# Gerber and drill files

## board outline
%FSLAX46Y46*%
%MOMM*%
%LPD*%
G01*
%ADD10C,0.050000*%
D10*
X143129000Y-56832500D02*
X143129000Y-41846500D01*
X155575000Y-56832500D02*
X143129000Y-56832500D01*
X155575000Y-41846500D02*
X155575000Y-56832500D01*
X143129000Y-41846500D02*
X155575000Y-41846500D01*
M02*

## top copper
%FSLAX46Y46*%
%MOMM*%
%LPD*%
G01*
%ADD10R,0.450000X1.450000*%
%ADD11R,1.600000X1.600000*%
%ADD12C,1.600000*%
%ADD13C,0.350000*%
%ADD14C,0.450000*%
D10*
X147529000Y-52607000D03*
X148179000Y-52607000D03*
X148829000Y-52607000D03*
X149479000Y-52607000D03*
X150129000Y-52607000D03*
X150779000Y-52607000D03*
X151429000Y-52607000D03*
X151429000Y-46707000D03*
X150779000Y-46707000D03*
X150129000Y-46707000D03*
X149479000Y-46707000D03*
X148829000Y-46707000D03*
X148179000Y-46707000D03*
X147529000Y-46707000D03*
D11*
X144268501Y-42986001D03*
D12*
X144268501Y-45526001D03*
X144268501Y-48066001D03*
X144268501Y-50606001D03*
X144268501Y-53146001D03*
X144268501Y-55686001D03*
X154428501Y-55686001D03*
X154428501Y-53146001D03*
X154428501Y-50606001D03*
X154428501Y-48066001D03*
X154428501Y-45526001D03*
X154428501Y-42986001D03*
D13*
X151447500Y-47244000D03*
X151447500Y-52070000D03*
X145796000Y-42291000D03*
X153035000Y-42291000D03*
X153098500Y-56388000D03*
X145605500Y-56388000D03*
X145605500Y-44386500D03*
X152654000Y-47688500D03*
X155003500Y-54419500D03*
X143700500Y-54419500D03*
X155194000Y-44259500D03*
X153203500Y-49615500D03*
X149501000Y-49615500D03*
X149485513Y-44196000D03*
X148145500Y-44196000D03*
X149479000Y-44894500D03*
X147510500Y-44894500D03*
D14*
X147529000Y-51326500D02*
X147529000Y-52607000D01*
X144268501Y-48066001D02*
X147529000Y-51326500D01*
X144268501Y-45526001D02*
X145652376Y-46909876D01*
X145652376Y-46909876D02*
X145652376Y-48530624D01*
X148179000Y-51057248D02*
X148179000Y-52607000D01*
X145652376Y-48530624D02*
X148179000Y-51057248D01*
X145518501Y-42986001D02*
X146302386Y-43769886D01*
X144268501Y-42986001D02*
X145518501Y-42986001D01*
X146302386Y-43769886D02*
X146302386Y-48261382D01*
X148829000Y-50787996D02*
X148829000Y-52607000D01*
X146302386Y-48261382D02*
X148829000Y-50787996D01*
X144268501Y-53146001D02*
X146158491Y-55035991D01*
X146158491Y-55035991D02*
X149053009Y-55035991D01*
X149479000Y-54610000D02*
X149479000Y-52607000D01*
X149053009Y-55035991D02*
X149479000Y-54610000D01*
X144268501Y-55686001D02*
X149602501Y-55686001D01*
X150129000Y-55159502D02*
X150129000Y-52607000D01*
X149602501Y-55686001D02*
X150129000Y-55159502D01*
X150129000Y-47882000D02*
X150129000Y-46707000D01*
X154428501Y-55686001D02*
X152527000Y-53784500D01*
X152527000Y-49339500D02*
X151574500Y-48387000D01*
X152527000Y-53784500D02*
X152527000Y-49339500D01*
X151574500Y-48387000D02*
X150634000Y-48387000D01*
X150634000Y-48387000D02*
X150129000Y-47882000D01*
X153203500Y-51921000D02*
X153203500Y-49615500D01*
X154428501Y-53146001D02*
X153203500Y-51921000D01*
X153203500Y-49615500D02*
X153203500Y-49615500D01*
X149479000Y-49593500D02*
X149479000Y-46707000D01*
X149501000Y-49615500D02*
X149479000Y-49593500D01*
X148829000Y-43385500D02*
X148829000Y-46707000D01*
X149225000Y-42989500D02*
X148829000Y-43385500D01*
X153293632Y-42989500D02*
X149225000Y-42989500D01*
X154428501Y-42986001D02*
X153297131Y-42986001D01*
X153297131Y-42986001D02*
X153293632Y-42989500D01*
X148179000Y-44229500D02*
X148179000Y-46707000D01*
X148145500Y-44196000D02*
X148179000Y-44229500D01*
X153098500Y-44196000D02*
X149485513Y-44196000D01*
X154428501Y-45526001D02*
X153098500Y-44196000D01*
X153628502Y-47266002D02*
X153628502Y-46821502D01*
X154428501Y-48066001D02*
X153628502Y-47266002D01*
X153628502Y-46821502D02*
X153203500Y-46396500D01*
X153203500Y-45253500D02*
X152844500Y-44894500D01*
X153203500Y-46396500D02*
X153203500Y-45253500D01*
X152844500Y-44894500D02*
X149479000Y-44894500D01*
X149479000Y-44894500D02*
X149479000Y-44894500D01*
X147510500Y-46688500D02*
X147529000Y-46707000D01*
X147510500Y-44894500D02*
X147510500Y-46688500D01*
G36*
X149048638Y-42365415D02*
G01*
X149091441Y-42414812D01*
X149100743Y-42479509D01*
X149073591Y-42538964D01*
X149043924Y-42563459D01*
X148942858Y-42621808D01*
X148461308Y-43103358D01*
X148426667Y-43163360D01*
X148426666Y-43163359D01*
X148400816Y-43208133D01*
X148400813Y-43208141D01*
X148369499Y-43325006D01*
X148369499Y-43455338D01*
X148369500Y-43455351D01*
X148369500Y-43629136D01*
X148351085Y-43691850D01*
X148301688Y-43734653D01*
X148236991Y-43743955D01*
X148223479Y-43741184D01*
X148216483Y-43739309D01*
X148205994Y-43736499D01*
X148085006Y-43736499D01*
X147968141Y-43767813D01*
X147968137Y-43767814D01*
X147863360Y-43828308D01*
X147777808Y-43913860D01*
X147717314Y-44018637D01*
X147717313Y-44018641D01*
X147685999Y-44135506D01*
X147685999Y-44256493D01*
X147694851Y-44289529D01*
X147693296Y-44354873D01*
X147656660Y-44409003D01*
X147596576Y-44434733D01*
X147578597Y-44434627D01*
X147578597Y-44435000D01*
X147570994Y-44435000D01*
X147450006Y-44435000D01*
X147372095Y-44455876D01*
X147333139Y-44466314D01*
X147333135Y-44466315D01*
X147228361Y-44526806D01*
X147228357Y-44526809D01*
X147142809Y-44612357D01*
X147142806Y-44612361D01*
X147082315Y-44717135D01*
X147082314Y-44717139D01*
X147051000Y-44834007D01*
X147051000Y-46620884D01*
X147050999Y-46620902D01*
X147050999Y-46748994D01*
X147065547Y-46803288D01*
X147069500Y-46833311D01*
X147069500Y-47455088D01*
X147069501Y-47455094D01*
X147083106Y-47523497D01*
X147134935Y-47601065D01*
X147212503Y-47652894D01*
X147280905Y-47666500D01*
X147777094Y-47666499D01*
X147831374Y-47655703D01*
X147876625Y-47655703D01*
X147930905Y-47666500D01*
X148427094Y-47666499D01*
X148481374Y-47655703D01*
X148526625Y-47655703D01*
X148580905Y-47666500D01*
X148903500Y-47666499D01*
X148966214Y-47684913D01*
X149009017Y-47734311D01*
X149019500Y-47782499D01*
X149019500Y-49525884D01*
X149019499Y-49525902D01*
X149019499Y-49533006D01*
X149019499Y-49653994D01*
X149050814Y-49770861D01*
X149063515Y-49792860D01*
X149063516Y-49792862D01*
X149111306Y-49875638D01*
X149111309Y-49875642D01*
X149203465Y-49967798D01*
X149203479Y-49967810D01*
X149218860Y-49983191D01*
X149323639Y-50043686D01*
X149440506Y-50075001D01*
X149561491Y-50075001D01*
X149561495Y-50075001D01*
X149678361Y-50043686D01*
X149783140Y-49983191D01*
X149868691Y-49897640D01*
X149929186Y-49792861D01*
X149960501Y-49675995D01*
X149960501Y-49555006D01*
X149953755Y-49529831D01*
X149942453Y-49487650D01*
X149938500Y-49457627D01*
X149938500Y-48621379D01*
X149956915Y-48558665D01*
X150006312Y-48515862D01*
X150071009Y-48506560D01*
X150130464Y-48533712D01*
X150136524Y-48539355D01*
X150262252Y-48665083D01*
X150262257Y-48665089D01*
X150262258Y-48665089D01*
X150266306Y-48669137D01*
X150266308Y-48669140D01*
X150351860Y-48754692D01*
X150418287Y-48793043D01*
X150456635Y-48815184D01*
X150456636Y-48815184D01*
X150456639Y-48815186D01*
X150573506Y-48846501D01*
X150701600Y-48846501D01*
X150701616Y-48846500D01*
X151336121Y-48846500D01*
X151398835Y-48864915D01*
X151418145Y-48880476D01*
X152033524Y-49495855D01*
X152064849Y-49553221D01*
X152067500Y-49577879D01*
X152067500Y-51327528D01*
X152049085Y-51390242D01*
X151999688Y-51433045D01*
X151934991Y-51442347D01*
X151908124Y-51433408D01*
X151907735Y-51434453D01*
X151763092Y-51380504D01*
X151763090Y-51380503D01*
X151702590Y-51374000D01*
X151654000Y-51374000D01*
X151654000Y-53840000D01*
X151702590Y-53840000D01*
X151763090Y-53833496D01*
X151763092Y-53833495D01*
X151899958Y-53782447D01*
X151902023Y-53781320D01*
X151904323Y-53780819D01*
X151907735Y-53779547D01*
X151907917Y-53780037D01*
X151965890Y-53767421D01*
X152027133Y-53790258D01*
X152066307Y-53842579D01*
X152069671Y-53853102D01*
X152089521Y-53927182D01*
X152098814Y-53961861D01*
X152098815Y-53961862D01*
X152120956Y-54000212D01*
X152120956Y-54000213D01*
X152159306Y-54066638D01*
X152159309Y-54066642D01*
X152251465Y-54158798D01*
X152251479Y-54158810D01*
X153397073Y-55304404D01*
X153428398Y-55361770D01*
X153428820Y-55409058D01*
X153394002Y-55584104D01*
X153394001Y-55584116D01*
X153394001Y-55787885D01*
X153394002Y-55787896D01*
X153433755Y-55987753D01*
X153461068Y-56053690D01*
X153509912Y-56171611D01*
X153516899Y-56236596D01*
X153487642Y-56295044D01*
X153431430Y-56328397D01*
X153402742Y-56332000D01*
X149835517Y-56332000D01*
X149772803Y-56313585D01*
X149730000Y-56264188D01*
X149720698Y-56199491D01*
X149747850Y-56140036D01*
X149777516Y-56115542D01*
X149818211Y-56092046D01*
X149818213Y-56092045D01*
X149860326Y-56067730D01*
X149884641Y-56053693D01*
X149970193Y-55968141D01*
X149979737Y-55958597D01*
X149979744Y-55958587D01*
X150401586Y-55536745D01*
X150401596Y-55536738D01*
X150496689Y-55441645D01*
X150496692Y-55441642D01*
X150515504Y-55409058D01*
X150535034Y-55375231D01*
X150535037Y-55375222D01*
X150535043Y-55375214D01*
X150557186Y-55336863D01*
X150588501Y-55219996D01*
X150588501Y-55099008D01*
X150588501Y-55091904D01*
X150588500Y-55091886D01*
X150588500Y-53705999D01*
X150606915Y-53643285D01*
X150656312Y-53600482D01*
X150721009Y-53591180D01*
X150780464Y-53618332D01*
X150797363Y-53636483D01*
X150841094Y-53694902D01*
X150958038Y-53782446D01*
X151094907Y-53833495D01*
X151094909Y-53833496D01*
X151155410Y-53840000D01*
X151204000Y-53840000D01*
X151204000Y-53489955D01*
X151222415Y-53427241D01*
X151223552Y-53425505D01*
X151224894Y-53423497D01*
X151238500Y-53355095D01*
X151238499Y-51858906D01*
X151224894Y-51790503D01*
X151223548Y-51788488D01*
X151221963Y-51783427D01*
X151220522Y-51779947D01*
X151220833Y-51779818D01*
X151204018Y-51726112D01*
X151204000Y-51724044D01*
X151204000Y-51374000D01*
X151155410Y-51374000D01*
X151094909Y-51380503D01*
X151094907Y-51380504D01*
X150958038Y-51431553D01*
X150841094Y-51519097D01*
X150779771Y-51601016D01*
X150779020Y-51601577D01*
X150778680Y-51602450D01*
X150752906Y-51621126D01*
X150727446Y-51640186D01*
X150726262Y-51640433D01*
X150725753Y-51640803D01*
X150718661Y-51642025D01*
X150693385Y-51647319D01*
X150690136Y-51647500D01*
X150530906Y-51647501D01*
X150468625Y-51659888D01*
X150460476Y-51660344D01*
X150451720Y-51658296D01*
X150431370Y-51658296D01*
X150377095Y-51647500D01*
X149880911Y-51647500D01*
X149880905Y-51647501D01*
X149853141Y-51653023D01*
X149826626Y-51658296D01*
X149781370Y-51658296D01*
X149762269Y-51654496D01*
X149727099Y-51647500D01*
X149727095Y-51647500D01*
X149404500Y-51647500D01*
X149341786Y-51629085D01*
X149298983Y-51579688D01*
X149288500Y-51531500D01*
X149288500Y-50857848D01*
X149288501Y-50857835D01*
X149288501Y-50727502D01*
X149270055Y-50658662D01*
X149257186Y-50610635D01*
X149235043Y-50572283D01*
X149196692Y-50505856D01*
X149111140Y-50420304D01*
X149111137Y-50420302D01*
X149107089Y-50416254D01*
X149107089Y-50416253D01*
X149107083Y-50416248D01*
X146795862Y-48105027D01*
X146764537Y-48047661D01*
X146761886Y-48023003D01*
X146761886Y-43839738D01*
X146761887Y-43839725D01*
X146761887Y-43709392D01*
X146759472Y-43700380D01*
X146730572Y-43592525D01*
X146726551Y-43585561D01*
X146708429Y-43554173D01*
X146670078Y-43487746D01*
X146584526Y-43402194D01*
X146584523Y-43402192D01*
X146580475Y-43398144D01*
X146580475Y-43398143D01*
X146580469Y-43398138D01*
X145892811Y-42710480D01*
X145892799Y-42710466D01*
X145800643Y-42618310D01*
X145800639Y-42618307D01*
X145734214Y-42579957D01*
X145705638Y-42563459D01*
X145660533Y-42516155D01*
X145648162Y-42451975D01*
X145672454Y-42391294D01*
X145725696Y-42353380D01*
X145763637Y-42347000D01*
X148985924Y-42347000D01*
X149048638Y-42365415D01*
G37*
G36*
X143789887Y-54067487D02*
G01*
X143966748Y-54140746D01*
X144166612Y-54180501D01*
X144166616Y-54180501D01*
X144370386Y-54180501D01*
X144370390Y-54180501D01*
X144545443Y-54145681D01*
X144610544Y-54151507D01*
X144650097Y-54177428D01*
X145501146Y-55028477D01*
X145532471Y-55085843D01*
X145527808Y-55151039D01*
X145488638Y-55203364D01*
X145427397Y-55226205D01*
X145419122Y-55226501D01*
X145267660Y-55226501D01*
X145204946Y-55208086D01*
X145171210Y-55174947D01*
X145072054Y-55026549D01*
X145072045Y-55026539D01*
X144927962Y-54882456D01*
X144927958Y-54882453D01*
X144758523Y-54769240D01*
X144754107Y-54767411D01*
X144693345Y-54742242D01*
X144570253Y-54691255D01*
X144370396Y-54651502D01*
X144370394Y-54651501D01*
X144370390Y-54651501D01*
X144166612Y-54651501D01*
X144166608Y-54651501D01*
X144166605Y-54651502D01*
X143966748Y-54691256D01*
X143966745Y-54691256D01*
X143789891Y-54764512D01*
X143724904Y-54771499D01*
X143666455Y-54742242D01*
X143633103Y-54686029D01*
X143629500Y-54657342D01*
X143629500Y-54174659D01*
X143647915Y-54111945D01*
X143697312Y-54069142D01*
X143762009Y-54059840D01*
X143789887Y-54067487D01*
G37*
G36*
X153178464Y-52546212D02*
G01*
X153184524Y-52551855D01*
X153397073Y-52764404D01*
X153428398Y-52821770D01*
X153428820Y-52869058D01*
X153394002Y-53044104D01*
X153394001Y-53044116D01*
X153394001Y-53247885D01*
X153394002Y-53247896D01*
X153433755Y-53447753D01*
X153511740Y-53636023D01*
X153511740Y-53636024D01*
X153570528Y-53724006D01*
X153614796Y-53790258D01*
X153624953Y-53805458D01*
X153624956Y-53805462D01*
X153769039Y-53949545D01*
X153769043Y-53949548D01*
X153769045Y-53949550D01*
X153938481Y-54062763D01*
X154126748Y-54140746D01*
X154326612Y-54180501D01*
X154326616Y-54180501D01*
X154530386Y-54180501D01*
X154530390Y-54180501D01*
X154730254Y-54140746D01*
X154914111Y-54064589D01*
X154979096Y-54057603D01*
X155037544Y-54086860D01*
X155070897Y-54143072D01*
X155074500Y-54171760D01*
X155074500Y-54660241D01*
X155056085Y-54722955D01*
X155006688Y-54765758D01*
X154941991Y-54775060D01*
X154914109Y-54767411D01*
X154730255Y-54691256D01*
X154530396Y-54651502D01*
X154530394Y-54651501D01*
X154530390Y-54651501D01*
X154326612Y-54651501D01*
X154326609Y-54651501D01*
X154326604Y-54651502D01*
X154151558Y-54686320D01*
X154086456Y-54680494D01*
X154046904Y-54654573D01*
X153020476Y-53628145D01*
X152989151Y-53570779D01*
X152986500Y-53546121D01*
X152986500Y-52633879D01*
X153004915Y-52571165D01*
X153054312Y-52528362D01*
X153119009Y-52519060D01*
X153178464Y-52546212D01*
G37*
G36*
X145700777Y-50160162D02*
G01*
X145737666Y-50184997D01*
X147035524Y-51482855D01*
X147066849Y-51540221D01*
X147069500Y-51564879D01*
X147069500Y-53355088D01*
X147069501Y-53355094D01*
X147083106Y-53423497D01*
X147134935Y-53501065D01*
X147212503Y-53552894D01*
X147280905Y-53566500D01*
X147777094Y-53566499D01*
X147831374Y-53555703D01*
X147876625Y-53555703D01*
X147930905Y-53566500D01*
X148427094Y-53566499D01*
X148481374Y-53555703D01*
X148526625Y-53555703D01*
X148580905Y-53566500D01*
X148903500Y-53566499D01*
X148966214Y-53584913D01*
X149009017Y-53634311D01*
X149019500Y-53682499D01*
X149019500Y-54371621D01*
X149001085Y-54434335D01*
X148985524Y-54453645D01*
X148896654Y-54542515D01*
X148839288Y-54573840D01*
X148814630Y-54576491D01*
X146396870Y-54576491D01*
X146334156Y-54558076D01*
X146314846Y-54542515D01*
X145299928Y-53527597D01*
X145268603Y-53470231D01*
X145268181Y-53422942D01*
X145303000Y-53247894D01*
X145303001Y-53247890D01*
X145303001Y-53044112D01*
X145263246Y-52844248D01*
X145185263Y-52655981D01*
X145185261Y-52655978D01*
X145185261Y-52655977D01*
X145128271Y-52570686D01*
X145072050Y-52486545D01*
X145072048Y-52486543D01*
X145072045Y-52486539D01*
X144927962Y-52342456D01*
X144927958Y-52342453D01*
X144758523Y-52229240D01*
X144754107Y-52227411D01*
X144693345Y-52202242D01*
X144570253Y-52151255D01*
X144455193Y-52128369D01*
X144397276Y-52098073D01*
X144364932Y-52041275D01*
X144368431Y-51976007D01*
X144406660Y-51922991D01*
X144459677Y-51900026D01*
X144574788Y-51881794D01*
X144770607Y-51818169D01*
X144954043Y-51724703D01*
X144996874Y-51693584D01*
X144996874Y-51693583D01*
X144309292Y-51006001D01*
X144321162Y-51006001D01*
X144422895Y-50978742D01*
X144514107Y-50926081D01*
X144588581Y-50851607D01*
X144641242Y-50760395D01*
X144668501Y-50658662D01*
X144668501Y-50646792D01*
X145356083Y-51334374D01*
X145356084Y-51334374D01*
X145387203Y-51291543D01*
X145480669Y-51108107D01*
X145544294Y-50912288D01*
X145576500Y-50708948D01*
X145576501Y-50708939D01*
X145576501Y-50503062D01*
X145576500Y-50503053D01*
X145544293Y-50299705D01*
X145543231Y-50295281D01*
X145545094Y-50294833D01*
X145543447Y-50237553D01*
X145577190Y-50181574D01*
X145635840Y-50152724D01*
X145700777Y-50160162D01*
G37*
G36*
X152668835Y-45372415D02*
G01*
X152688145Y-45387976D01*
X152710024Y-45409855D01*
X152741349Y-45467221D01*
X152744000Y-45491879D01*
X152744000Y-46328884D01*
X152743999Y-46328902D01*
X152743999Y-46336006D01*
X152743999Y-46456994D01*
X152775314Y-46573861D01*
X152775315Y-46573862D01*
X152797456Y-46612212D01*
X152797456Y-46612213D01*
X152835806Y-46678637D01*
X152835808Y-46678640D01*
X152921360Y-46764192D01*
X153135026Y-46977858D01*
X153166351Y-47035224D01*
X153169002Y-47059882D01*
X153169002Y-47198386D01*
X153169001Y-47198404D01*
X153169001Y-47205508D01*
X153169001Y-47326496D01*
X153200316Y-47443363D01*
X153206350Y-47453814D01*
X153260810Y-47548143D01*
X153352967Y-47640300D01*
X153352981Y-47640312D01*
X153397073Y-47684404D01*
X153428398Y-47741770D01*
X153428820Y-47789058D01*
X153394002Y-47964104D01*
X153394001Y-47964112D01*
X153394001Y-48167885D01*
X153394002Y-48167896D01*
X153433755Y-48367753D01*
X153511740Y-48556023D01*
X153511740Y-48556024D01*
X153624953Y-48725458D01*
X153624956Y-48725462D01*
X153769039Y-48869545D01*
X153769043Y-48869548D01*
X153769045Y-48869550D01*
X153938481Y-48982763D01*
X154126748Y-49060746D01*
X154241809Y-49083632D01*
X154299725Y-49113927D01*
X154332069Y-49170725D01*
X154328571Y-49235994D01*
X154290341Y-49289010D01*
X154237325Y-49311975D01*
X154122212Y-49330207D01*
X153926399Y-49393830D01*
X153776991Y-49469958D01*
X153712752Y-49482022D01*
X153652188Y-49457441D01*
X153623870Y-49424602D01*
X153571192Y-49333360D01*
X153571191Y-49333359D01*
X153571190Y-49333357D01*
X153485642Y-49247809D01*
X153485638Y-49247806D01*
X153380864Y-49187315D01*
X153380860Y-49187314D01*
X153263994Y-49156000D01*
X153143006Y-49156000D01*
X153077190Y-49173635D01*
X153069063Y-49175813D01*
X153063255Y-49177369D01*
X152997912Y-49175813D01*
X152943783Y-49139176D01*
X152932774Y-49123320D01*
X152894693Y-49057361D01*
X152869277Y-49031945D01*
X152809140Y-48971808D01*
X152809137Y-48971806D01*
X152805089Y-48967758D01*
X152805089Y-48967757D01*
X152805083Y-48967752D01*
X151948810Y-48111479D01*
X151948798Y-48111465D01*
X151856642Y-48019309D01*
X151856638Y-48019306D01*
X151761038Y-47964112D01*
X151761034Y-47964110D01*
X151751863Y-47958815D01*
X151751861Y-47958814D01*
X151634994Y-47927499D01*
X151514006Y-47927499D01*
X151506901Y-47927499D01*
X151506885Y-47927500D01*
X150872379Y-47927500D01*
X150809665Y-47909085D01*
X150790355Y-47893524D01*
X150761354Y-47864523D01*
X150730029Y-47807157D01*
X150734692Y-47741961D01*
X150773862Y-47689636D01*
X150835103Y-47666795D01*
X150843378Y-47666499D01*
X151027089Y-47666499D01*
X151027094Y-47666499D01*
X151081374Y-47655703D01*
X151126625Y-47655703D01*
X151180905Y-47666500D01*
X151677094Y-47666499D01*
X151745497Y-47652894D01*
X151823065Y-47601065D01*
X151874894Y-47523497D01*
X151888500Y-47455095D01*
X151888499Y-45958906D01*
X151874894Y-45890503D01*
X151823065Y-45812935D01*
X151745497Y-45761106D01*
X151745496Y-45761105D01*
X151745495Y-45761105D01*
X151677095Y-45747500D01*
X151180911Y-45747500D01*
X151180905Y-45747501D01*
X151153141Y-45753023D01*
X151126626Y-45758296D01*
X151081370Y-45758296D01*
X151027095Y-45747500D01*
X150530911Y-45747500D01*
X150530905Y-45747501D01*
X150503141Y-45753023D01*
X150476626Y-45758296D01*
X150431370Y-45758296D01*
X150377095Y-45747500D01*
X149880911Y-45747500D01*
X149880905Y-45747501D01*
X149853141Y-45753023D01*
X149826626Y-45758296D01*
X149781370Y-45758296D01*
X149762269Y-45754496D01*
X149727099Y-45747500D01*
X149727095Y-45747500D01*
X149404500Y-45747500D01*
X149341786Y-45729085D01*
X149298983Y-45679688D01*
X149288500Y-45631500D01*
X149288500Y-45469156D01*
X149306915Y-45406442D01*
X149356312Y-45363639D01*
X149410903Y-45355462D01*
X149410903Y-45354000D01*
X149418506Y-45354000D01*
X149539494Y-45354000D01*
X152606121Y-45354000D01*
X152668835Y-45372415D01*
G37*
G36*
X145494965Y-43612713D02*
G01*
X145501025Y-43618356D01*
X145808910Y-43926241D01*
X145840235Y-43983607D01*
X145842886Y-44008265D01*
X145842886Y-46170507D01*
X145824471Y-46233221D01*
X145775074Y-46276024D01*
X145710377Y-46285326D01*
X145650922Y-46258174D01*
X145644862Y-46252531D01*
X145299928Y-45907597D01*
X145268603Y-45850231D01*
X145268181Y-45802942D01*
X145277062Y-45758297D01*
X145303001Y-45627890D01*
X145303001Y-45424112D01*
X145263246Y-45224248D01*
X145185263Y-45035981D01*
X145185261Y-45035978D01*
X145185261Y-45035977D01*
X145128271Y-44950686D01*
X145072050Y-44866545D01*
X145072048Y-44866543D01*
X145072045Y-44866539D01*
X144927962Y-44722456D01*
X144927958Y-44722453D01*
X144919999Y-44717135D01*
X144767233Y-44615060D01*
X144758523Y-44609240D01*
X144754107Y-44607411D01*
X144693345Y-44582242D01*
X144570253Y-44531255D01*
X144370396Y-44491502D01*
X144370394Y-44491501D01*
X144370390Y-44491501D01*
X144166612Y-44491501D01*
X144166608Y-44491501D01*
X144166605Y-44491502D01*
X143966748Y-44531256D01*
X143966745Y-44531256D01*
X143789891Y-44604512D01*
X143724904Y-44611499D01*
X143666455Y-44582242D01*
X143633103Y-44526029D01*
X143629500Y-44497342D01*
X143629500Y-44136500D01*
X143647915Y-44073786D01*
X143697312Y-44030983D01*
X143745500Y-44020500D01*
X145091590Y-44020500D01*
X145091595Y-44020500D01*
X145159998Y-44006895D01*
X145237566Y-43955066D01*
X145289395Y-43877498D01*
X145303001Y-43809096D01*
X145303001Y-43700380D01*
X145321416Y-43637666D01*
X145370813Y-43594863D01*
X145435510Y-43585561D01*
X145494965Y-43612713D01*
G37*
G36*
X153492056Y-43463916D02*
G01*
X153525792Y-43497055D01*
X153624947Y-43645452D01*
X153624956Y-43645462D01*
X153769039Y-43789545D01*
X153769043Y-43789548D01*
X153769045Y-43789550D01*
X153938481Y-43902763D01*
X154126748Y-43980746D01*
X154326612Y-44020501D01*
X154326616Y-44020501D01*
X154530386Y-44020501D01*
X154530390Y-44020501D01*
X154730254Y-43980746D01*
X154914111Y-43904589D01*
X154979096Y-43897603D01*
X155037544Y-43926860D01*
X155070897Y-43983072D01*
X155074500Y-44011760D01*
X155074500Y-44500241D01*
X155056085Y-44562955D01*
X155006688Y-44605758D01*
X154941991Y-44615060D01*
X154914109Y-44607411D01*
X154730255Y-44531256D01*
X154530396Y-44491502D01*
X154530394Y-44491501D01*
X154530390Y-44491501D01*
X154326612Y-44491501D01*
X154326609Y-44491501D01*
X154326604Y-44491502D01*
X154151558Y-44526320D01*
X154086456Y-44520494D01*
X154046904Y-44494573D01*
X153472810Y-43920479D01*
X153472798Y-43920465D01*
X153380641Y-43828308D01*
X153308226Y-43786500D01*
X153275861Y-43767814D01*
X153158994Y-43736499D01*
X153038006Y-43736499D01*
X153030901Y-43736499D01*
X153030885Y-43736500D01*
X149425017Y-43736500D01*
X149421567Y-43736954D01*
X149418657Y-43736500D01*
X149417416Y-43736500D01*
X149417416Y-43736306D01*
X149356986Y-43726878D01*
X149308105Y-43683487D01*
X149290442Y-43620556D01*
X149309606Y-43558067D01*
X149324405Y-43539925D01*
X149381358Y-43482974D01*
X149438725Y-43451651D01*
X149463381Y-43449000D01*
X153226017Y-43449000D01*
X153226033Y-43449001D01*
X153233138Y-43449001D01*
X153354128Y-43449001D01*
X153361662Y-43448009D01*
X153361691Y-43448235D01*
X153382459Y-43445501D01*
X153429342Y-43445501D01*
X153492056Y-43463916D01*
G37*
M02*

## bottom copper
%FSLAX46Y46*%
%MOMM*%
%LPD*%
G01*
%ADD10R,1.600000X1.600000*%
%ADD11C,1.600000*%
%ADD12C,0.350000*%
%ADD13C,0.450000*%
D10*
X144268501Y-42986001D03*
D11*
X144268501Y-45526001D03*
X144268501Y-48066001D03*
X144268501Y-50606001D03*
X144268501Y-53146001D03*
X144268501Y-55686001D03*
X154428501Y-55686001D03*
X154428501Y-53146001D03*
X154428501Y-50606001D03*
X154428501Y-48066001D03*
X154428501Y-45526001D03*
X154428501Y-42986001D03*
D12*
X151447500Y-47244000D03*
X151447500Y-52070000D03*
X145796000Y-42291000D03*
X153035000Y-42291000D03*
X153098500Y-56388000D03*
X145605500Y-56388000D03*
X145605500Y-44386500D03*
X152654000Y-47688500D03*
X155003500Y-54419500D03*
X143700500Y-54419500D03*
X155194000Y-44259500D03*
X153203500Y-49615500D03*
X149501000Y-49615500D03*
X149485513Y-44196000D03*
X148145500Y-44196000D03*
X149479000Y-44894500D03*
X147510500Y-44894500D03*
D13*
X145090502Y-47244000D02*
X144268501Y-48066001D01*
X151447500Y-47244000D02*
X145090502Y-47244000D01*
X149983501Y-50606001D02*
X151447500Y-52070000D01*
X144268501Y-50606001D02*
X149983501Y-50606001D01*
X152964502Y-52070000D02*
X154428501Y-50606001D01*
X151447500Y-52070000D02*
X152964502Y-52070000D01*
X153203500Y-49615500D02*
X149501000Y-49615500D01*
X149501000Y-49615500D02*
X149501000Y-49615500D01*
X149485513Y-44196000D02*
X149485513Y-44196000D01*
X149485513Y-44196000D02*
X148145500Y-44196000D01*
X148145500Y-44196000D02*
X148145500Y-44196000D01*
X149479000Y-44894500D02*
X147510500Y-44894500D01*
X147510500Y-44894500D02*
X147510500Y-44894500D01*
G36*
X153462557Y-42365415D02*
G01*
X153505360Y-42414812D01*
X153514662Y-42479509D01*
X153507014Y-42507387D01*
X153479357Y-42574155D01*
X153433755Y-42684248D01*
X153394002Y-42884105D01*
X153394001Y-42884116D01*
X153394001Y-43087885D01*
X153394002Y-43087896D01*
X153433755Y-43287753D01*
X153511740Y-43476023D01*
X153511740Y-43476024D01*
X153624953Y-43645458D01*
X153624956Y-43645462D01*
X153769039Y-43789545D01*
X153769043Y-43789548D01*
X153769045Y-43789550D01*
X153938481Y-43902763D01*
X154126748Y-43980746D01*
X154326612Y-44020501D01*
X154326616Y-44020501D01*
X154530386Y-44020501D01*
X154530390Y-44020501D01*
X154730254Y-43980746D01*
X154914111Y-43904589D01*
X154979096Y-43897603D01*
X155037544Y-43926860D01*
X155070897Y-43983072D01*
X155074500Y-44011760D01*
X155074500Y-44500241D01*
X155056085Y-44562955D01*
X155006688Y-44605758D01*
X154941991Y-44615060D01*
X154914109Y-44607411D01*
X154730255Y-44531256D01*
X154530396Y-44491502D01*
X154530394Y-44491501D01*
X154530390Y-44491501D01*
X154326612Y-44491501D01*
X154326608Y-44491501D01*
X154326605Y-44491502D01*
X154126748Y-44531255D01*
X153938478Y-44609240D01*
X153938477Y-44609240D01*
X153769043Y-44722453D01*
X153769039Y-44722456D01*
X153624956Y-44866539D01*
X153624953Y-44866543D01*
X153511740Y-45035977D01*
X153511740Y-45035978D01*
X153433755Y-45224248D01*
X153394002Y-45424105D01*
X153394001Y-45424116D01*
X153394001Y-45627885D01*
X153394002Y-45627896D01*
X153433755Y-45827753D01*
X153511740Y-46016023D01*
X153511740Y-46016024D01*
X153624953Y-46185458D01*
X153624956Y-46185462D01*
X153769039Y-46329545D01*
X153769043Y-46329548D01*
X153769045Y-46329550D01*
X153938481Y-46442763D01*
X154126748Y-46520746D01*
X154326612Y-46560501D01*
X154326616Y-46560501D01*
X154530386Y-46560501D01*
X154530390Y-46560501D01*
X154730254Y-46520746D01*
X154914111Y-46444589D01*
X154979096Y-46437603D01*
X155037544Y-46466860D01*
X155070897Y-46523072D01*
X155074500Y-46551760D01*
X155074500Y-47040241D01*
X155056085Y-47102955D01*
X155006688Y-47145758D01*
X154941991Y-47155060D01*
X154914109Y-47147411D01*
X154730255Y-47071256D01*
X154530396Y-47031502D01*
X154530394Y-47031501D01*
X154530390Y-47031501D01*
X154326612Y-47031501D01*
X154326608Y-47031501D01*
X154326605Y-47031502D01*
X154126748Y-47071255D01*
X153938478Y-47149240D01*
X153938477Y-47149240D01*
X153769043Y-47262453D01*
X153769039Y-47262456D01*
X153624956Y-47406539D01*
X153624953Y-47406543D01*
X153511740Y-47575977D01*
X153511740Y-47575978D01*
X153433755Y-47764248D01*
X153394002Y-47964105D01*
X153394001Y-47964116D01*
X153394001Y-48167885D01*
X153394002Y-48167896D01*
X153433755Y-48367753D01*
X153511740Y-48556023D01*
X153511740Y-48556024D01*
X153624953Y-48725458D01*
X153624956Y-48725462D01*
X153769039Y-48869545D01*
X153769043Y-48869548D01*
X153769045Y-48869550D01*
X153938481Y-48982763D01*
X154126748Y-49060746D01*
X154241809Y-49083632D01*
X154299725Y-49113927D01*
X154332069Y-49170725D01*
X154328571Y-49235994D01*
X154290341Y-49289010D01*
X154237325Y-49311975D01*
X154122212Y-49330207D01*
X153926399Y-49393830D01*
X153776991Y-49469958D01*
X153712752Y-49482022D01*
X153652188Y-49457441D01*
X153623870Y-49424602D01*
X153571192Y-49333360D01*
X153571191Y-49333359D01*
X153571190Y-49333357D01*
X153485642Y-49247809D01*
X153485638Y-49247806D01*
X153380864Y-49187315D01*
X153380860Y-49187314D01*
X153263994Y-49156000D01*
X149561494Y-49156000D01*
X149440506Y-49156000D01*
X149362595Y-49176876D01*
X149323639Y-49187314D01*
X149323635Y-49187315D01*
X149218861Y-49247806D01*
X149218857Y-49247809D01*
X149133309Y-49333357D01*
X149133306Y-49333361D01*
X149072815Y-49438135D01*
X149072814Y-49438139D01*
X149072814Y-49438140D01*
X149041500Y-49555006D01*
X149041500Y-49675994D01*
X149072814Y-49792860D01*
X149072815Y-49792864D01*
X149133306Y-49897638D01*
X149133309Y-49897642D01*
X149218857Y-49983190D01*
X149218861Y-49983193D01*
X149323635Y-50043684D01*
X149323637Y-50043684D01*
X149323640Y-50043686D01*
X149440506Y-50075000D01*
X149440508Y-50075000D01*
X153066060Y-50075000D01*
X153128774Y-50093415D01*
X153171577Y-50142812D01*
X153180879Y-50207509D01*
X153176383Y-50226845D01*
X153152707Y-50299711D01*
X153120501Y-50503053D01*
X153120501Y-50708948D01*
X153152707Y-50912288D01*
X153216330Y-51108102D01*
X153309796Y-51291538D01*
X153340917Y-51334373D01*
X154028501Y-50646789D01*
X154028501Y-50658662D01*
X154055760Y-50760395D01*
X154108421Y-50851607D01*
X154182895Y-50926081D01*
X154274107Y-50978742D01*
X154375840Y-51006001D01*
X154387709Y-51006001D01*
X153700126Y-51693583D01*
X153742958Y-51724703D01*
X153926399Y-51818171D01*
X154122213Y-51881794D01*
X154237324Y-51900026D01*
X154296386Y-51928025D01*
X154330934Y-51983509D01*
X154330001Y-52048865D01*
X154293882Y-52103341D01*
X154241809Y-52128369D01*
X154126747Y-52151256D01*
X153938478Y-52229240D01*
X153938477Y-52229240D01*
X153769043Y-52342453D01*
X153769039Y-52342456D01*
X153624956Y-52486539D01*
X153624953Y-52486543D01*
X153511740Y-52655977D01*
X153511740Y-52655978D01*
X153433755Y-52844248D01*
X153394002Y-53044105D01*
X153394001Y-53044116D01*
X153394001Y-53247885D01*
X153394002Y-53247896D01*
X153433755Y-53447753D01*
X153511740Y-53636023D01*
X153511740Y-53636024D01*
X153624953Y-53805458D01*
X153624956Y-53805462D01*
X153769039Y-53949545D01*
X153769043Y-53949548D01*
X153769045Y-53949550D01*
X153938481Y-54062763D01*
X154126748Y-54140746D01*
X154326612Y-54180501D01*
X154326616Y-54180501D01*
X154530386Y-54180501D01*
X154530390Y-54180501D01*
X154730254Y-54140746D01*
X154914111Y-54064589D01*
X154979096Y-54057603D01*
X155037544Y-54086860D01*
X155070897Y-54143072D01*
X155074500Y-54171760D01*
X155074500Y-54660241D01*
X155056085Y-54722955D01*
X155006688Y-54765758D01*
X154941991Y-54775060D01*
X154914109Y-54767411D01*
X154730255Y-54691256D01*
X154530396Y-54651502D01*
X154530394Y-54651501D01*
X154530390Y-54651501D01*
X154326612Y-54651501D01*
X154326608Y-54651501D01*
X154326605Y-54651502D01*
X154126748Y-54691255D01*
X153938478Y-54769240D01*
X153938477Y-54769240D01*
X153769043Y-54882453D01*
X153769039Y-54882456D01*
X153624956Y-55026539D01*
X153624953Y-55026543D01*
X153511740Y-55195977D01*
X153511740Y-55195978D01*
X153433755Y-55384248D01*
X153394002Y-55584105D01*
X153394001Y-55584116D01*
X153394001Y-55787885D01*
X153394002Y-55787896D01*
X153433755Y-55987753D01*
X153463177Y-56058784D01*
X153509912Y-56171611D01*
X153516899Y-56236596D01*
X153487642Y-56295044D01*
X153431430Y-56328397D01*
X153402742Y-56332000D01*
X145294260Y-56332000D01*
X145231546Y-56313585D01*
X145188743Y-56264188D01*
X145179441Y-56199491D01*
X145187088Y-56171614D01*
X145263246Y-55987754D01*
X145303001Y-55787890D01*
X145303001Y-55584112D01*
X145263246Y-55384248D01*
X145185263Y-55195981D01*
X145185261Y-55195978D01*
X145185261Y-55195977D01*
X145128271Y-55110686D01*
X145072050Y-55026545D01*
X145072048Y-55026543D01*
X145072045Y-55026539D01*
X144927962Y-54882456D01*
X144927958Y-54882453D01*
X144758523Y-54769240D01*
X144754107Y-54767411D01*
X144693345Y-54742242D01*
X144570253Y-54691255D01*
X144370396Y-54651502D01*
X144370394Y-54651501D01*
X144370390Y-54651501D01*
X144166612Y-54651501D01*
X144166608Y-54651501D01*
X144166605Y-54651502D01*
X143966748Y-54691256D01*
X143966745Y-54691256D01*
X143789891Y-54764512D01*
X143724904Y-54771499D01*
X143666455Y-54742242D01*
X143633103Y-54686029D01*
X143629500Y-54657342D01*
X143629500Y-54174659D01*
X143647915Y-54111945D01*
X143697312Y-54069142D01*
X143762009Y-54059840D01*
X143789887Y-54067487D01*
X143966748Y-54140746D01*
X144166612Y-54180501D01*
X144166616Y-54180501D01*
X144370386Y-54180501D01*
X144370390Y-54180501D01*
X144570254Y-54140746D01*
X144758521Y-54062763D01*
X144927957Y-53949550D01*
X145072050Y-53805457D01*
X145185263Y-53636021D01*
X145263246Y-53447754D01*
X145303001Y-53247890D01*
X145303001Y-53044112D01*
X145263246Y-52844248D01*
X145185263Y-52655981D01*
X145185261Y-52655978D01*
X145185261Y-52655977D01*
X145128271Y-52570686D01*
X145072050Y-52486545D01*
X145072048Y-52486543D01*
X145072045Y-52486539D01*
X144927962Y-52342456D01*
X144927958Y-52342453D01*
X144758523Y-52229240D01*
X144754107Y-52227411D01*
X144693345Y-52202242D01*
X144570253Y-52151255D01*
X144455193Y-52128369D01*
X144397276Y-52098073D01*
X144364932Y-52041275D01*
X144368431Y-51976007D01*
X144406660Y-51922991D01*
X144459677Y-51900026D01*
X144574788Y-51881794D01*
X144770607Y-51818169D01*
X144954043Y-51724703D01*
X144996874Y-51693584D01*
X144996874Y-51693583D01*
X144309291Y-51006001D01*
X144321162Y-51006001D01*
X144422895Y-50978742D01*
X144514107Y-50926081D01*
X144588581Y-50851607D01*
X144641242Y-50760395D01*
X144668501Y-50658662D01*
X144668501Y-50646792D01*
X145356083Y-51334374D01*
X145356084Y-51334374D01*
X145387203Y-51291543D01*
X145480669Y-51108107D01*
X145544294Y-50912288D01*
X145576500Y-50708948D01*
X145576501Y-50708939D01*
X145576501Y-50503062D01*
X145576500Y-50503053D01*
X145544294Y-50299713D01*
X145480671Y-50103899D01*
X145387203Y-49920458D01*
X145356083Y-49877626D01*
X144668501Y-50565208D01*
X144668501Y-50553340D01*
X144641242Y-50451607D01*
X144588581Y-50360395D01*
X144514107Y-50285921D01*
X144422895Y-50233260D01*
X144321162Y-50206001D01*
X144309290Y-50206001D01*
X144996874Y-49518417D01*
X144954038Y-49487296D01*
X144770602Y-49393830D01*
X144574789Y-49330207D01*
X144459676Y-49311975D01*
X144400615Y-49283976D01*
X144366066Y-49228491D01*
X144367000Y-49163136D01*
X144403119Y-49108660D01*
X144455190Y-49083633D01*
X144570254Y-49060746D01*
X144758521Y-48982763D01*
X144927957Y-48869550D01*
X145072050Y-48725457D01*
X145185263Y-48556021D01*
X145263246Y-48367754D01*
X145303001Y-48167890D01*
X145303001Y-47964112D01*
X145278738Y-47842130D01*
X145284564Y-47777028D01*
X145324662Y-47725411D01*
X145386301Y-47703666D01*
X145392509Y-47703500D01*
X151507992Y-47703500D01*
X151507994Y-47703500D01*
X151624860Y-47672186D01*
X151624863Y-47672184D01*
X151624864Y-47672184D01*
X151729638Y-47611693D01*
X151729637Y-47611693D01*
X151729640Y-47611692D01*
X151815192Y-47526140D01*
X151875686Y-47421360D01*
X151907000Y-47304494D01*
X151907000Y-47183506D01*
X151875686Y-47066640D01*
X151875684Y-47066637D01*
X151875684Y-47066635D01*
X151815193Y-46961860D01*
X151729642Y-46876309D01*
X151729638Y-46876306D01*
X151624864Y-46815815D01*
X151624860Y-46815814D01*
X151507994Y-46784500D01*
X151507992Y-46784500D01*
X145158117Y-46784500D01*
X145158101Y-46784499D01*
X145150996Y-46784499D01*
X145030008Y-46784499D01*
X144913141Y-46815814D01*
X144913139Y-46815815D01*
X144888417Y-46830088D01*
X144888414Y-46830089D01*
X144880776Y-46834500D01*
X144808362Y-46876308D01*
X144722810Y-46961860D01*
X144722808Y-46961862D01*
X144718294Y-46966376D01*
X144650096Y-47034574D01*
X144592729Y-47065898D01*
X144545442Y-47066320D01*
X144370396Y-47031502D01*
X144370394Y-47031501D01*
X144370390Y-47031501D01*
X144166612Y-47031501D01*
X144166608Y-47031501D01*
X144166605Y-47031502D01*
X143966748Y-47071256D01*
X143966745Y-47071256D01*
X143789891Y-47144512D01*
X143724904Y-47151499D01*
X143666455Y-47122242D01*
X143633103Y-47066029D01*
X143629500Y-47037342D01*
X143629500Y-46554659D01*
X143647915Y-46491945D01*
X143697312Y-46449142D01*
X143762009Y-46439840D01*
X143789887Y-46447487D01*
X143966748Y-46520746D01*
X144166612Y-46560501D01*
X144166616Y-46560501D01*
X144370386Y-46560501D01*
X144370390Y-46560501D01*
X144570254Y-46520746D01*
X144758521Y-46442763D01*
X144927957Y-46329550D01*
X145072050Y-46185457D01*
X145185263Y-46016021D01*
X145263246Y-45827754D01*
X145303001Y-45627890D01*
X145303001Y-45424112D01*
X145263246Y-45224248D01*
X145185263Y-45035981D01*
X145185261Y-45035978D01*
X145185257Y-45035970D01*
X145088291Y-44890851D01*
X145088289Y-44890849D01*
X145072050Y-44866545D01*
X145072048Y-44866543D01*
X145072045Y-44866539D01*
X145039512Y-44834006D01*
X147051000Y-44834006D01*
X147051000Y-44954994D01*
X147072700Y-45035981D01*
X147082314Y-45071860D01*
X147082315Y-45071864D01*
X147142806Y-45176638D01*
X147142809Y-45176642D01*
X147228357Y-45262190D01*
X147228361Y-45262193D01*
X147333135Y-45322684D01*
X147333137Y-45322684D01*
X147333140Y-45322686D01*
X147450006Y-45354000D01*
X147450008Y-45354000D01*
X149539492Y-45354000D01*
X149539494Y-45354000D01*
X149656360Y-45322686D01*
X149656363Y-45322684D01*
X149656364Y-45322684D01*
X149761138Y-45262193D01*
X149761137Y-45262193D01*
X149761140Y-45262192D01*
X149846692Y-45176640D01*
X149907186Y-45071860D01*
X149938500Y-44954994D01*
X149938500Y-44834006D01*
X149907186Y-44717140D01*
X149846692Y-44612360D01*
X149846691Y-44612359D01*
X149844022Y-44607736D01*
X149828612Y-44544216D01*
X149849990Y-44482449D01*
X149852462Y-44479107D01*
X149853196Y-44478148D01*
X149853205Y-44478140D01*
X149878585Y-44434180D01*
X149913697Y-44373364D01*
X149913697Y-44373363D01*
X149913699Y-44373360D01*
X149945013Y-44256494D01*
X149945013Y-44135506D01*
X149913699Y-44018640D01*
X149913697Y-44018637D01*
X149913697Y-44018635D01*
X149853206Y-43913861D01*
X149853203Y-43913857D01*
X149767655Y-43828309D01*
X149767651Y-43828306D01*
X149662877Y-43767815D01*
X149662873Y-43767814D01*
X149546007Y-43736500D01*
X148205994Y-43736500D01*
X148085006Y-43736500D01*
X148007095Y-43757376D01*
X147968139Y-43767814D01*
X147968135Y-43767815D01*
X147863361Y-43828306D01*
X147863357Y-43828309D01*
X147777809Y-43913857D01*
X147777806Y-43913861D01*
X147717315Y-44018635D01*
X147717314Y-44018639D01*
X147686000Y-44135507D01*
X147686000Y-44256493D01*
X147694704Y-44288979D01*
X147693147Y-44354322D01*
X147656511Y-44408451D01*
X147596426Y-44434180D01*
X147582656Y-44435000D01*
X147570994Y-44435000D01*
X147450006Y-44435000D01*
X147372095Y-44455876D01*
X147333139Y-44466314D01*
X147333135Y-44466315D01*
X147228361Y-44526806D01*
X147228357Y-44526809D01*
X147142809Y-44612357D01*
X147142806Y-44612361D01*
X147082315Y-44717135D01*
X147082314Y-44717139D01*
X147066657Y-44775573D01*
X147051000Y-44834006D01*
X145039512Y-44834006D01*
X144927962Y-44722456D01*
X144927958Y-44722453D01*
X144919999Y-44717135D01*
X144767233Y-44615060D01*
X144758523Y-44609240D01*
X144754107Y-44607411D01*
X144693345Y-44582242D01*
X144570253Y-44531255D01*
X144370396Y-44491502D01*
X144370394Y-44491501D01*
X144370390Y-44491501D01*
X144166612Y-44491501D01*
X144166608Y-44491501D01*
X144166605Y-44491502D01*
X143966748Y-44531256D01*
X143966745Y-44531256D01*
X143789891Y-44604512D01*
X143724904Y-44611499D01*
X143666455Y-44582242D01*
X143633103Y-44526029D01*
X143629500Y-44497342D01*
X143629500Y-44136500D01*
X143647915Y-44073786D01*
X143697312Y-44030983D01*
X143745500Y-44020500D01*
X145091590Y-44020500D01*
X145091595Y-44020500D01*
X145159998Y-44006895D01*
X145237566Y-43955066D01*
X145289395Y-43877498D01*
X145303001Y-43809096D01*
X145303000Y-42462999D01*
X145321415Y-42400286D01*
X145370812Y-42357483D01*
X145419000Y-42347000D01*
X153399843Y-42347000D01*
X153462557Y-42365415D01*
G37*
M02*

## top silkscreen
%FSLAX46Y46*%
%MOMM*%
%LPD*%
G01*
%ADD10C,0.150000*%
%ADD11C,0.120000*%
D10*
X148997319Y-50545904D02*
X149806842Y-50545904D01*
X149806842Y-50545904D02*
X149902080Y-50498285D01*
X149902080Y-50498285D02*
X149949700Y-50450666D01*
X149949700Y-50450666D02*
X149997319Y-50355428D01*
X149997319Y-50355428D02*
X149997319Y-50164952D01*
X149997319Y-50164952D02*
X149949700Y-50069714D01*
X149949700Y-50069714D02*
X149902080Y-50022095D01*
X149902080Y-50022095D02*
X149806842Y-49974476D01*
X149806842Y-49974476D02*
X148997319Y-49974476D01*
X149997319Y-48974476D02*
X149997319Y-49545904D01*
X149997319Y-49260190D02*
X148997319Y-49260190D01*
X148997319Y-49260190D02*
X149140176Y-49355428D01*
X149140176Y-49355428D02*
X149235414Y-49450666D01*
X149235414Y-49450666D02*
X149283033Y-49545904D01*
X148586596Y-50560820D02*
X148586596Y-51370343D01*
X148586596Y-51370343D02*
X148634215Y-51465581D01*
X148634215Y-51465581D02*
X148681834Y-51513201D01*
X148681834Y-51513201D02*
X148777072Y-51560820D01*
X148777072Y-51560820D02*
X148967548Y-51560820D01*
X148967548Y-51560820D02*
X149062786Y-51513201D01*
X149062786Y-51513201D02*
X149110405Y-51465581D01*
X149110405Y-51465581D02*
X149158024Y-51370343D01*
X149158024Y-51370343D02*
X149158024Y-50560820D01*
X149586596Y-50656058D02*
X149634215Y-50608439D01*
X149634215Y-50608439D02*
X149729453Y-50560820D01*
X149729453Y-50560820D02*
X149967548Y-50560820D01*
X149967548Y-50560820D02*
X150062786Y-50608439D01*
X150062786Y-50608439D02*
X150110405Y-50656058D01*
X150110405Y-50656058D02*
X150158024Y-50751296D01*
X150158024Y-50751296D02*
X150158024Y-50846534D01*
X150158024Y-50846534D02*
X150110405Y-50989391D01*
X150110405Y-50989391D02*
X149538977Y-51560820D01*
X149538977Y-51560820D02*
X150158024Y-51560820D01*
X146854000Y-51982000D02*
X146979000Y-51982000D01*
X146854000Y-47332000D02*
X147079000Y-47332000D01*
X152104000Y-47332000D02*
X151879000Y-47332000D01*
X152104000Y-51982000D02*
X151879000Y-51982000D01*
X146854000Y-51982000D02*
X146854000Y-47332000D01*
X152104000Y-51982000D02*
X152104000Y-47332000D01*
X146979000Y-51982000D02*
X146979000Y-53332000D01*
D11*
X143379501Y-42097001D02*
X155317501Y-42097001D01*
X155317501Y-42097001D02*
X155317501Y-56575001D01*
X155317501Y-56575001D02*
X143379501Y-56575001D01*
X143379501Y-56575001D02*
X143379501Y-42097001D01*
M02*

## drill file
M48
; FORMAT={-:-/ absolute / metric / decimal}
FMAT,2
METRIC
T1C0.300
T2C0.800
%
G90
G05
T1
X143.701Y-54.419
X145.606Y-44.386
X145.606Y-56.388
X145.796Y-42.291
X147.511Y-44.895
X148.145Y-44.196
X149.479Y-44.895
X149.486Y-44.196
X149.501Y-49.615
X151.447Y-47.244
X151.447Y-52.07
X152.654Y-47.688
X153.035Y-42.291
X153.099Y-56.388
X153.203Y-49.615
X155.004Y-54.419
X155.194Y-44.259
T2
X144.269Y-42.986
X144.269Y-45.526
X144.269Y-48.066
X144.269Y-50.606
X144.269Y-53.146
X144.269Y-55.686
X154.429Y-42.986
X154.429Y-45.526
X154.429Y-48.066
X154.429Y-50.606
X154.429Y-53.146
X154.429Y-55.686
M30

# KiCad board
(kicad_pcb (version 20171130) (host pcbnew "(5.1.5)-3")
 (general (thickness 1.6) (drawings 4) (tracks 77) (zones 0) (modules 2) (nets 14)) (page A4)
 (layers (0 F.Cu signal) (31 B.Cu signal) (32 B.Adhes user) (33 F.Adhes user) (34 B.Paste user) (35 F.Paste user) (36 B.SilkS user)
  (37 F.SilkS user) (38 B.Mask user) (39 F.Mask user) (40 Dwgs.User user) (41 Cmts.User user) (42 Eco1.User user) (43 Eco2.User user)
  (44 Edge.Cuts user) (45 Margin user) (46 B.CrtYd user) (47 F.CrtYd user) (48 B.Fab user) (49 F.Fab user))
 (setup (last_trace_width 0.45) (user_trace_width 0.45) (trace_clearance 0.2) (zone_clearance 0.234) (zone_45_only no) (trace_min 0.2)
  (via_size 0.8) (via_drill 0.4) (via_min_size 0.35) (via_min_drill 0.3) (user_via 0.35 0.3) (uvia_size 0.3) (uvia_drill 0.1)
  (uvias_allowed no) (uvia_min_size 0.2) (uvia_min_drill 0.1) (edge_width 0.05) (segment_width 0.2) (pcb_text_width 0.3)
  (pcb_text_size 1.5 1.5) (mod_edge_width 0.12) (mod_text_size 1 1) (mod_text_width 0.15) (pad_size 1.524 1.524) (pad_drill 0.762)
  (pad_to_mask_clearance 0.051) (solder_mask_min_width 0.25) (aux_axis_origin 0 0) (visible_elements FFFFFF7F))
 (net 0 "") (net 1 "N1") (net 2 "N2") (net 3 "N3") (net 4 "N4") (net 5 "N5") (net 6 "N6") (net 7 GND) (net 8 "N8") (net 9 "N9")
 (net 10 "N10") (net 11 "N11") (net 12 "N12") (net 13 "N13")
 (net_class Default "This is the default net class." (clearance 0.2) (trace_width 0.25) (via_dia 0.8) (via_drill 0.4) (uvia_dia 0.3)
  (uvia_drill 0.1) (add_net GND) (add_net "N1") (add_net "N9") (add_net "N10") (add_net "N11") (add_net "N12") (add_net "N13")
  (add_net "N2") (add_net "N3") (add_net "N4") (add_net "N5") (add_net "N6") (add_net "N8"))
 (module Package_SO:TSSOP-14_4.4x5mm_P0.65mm (layer F.Cu) (at 149.479 49.657 90)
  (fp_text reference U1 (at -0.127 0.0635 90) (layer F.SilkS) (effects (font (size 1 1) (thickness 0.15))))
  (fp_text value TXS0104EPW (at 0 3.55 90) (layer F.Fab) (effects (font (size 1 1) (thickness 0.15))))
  (fp_line (start -2.325 -2.625) (end -2.325 -2.5) (layer F.SilkS) (width 0.15))
  (fp_line (start 2.325 -2.625) (end 2.325 -2.4) (layer F.SilkS) (width 0.15))
  (fp_line (start 2.325 2.625) (end 2.325 2.4) (layer F.SilkS) (width 0.15))
  (fp_line (start -2.325 2.625) (end -2.325 2.4) (layer F.SilkS) (width 0.15))
  (fp_line (start -2.325 -2.625) (end 2.325 -2.625) (layer F.SilkS) (width 0.15))
  (fp_line (start -2.325 2.625) (end 2.325 2.625) (layer F.SilkS) (width 0.15))
  (fp_line (start -2.325 -2.5) (end -3.675 -2.5) (layer F.SilkS) (width 0.15))
  (pad 1 smd rect (at -2.95 -1.95 90) (size 1.45 0.45) (layers F.Cu F.Paste F.Mask) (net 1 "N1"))
  (pad 2 smd rect (at -2.95 -1.3 90) (size 1.45 0.45) (layers F.Cu F.Paste F.Mask) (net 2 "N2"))
  (pad 3 smd rect (at -2.95 -0.65 90) (size 1.45 0.45) (layers F.Cu F.Paste F.Mask) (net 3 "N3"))
  (pad 4 smd rect (at -2.95 0 90) (size 1.45 0.45) (layers F.Cu F.Paste F.Mask) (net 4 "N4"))
  (pad 5 smd rect (at -2.95 0.65 90) (size 1.45 0.45) (layers F.Cu F.Paste F.Mask) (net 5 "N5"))
  (pad 6 smd rect (at -2.95 1.3 90) (size 1.45 0.45) (layers F.Cu F.Paste F.Mask) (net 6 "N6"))
  (pad 7 smd rect (at -2.95 1.95 90) (size 1.45 0.45) (layers F.Cu F.Paste F.Mask) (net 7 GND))
  (pad 8 smd rect (at 2.95 1.95 90) (size 1.45 0.45) (layers F.Cu F.Paste F.Mask) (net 1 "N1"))
  (pad 9 smd rect (at 2.95 1.3 90) (size 1.45 0.45) (layers F.Cu F.Paste F.Mask) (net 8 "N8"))
  (pad 10 smd rect (at 2.95 0.65 90) (size 1.45 0.45) (layers F.Cu F.Paste F.Mask) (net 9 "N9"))
  (pad 11 smd rect (at 2.95 0 90) (size 1.45 0.45) (layers F.Cu F.Paste F.Mask) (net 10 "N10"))
  (pad 12 smd rect (at 2.95 -0.65 90) (size 1.45 0.45) (layers F.Cu F.Paste F.Mask) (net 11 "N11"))
  (pad 13 smd rect (at 2.95 -1.3 90) (size 1.45 0.45) (layers F.Cu F.Paste F.Mask) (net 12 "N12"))
  (pad 14 smd rect (at 2.95 -1.95 90) (size 1.45 0.45) (layers F.Cu F.Paste F.Mask) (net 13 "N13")))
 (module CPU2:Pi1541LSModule (layer F.Cu) (at 149.348501 50.606001)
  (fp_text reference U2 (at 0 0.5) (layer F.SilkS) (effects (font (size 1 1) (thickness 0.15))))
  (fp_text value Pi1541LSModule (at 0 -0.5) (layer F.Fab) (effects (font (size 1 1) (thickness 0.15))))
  (fp_line (start -5.969 -8.509) (end 5.969 -8.509) (layer F.SilkS) (width 0.12))
  (fp_line (start 5.969 -8.509) (end 5.969 5.969) (layer F.SilkS) (width 0.12))
  (fp_line (start 5.969 5.969) (end -5.969 5.969) (layer F.SilkS) (width 0.12))
  (fp_line (start -5.969 5.969) (end -5.969 -8.509) (layer F.SilkS) (width 0.12))
  (pad 1 thru_hole rect (at -5.08 -7.62) (size 1.6 1.6) (drill 0.8) (layers *.Cu *.Mask) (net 3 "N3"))
  (pad 2 thru_hole circle (at -5.08 -5.08) (size 1.6 1.6) (drill 0.8) (layers *.Cu *.Mask) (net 2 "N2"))
  (pad 3 thru_hole circle (at -5.08 -2.54) (size 1.6 1.6) (drill 0.8) (layers *.Cu *.Mask) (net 1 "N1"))
  (pad 4 thru_hole circle (at -5.08 0) (size 1.6 1.6) (drill 0.8) (layers *.Cu *.Mask) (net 7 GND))
  (pad 5 thru_hole circle (at -5.08 2.54) (size 1.6 1.6) (drill 0.8) (layers *.Cu *.Mask) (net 4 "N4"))
  (pad 6 thru_hole circle (at -5.08 5.08) (size 1.6 1.6) (drill 0.8) (layers *.Cu *.Mask) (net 5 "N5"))
  (pad 7 thru_hole circle (at 5.08 5.08) (size 1.6 1.6) (drill 0.8) (layers *.Cu *.Mask) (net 9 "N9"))
  (pad 8 thru_hole circle (at 5.08 2.54) (size 1.6 1.6) (drill 0.8) (layers *.Cu *.Mask) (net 10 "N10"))
  (pad 9 thru_hole circle (at 5.08 0) (size 1.6 1.6) (drill 0.8) (layers *.Cu *.Mask) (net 7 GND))
  (pad 10 thru_hole circle (at 5.08 -2.54) (size 1.6 1.6) (drill 0.8) (layers *.Cu *.Mask) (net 13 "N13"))
  (pad 11 thru_hole circle (at 5.08 -5.08) (size 1.6 1.6) (drill 0.8) (layers *.Cu *.Mask) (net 12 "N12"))
  (pad 12 thru_hole circle (at 5.08 -7.62) (size 1.6 1.6) (drill 0.8) (layers *.Cu *.Mask) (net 11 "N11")))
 (gr_line (start 143.129 56.8325) (end 143.129 41.8465) (layer Edge.Cuts) (width 0.05))
 (gr_line (start 155.575 56.8325) (end 143.129 56.8325) (layer Edge.Cuts) (width 0.05))
 (gr_line (start 155.575 41.8465) (end 155.575 56.8325) (layer Edge.Cuts) (width 0.05))
 (gr_line (start 143.129 41.8465) (end 155.575 41.8465) (layer Edge.Cuts) (width 0.05))
 (via (at 151.4475 47.244) (size 0.35) (drill 0.3) (layers F.Cu B.Cu) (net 1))
 (segment (start 147.529 51.3265) (end 147.529 52.607) (width 0.45) (layer F.Cu) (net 1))
 (segment (start 144.268501 48.066001) (end 147.529 51.3265) (width 0.45) (layer F.Cu) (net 1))
 (segment (start 145.090502 47.244) (end 144.268501 48.066001) (width 0.45) (layer B.Cu) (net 1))
 (segment (start 151.4475 47.244) (end 145.090502 47.244) (width 0.45) (layer B.Cu) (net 1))
 (segment (start 144.268501 45.526001) (end 145.652376 46.909876) (width 0.45) (layer F.Cu) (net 2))
 (segment (start 145.652376 46.909876) (end 145.652376 48.530624) (width 0.45) (layer F.Cu) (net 2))
 (segment (start 148.179 51.057248) (end 148.179 52.607) (width 0.45) (layer F.Cu) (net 2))
 (segment (start 145.652376 48.530624) (end 148.179 51.057248) (width 0.45) (layer F.Cu) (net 2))
 (segment (start 145.518501 42.986001) (end 146.302386 43.769886) (width 0.45) (layer F.Cu) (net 3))
 (segment (start 144.268501 42.986001) (end 145.518501 42.986001) (width 0.45) (layer F.Cu) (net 3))
 (segment (start 146.302386 43.769886) (end 146.302386 48.261382) (width 0.45) (layer F.Cu) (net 3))
 (segment (start 148.829 50.787996) (end 148.829 52.607) (width 0.45) (layer F.Cu) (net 3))
 (segment (start 146.302386 48.261382) (end 148.829 50.787996) (width 0.45) (layer F.Cu) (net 3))
 (via (at 151.4475 52.07) (size 0.35) (drill 0.3) (layers F.Cu B.Cu) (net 7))
 (segment (start 144.268501 53.146001) (end 146.158491 55.035991) (width 0.45) (layer F.Cu) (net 4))
 (segment (start 146.158491 55.035991) (end 149.053009 55.035991) (width 0.45) (layer F.Cu) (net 4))
 (segment (start 149.479 54.61) (end 149.479 52.607) (width 0.45) (layer F.Cu) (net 4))
 (segment (start 149.053009 55.035991) (end 149.479 54.61) (width 0.45) (layer F.Cu) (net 4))
 (segment (start 144.268501 55.686001) (end 149.602501 55.686001) (width 0.45) (layer F.Cu) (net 5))
 (segment (start 150.129 55.159502) (end 150.129 52.607) (width 0.45) (layer F.Cu) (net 5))
 (segment (start 149.602501 55.686001) (end 150.129 55.159502) (width 0.45) (layer F.Cu) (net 5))
 (segment (start 149.983501 50.606001) (end 151.4475 52.07) (width 0.45) (layer B.Cu) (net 7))
 (segment (start 144.268501 50.606001) (end 149.983501 50.606001) (width 0.45) (layer B.Cu) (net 7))
 (segment (start 152.964502 52.07) (end 154.428501 50.606001) (width 0.45) (layer B.Cu) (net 7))
 (segment (start 151.4475 52.07) (end 152.964502 52.07) (width 0.45) (layer B.Cu) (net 7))
 (via (at 145.796 42.291) (size 0.35) (drill 0.3) (layers F.Cu B.Cu) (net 7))
 (via (at 153.035 42.291) (size 0.35) (drill 0.3) (layers F.Cu B.Cu) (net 7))
 (via (at 153.0985 56.388) (size 0.35) (drill 0.3) (layers F.Cu B.Cu) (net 7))
 (via (at 145.6055 56.388) (size 0.35) (drill 0.3) (layers F.Cu B.Cu) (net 7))
 (via (at 145.6055 44.3865) (size 0.35) (drill 0.3) (layers F.Cu B.Cu) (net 7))
 (via (at 152.654 47.6885) (size 0.35) (drill 0.3) (layers F.Cu B.Cu) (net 7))
 (via (at 155.0035 54.4195) (size 0.35) (drill 0.3) (layers F.Cu B.Cu) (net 7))
 (via (at 143.7005 54.4195) (size 0.35) (drill 0.3) (layers F.Cu B.Cu) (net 7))
 (via (at 155.194 44.2595) (size 0.35) (drill 0.3) (layers F.Cu B.Cu) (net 7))
 (segment (start 150.129 47.882) (end 150.129 46.707) (width 0.45) (layer F.Cu) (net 9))
 (segment (start 154.428501 55.686001) (end 152.527 53.7845) (width 0.45) (layer F.Cu) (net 9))
 (segment (start 152.527 49.3395) (end 151.5745 48.387) (width 0.45) (layer F.Cu) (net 9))
 (segment (start 152.527 53.7845) (end 152.527 49.3395) (width 0.45) (layer F.Cu) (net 9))
 (segment (start 151.5745 48.387) (end 150.634 48.387) (width 0.45) (layer F.Cu) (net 9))
 (segment (start 150.634 48.387) (end 150.129 47.882) (width 0.45) (layer F.Cu) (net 9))
 (segment (start 153.2035 51.921) (end 153.2035 49.6155) (width 0.45) (layer F.Cu) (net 10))
 (segment (start 154.428501 53.146001) (end 153.2035 51.921) (width 0.45) (layer F.Cu) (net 10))
 (segment (start 153.2035 49.6155) (end 153.2035 49.6155) (width 0.45) (layer F.Cu) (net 10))
 (via (at 153.2035 49.6155) (size 0.35) (drill 0.3) (layers F.Cu B.Cu) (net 10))
 (segment (start 153.2035 49.6155) (end 149.501 49.6155) (width 0.45) (layer B.Cu) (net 10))
 (segment (start 149.501 49.6155) (end 149.501 49.6155) (width 0.45) (layer B.Cu) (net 10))
 (via (at 149.501 49.6155) (size 0.35) (drill 0.3) (layers F.Cu B.Cu) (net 10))
 (segment (start 149.479 49.5935) (end 149.479 46.707) (width 0.45) (layer F.Cu) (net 10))
 (segment (start 149.501 49.6155) (end 149.479 49.5935) (width 0.45) (layer F.Cu) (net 10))
 (segment (start 148.829 43.3855) (end 148.829 46.707) (width 0.45) (layer F.Cu) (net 11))
 (segment (start 149.225 42.9895) (end 148.829 43.3855) (width 0.45) (layer F.Cu) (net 11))
 (segment (start 153.293632 42.9895) (end 149.225 42.9895) (width 0.45) (layer F.Cu) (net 11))
 (segment (start 154.428501 42.986001) (end 153.297131 42.986001) (width 0.45) (layer F.Cu) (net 11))
 (segment (start 153.297131 42.986001) (end 153.293632 42.9895) (width 0.45) (layer F.Cu) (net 11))
 (segment (start 149.485513 44.196) (end 149.485513 44.196) (width 0.45) (layer B.Cu) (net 12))
 (segment (start 149.485513 44.196) (end 148.1455 44.196) (width 0.45) (layer B.Cu) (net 12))
 (via (at 149.485513 44.196) (size 0.35) (drill 0.3) (layers F.Cu B.Cu) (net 12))
 (segment (start 148.1455 44.196) (end 148.1455 44.196) (width 0.45) (layer B.Cu) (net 12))
 (via (at 148.1455 44.196) (size 0.35) (drill 0.3) (layers F.Cu B.Cu) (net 12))
 (segment (start 148.179 44.2295) (end 148.179 46.707) (width 0.45) (layer F.Cu) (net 12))
 (segment (start 148.1455 44.196) (end 148.179 44.2295) (width 0.45) (layer F.Cu) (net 12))
 (segment (start 153.0985 44.196) (end 149.485513 44.196) (width 0.45) (layer F.Cu) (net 12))
 (segment (start 154.428501 45.526001) (end 153.0985 44.196) (width 0.45) (layer F.Cu) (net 12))
 (segment (start 153.628502 47.266002) (end 153.628502 46.821502) (width 0.45) (layer F.Cu) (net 13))
 (segment (start 154.428501 48.066001) (end 153.628502 47.266002) (width 0.45) (layer F.Cu) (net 13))
 (segment (start 153.628502 46.821502) (end 153.2035 46.3965) (width 0.45) (layer F.Cu) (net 13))
 (segment (start 153.2035 45.2535) (end 152.8445 44.8945) (width 0.45) (layer F.Cu) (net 13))
 (segment (start 153.2035 46.3965) (end 153.2035 45.2535) (width 0.45) (layer F.Cu) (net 13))
 (segment (start 152.8445 44.8945) (end 149.479 44.8945) (width 0.45) (layer F.Cu) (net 13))
 (segment (start 149.479 44.8945) (end 149.479 44.8945) (width 0.45) (layer F.Cu) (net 13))
 (via (at 149.479 44.8945) (size 0.35) (drill 0.3) (layers F.Cu B.Cu) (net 13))
 (segment (start 149.479 44.8945) (end 147.5105 44.8945) (width 0.45) (layer B.Cu) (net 13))
 (segment (start 147.5105 44.8945) (end 147.5105 44.8945) (width 0.45) (layer B.Cu) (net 13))
 (via (at 147.5105 44.8945) (size 0.35) (drill 0.3) (layers F.Cu B.Cu) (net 13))
 (segment (start 147.5105 46.6885) (end 147.529 46.707) (width 0.45) (layer F.Cu) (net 13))
 (segment (start 147.5105 44.8945) (end 147.5105 46.6885) (width 0.45) (layer F.Cu) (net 13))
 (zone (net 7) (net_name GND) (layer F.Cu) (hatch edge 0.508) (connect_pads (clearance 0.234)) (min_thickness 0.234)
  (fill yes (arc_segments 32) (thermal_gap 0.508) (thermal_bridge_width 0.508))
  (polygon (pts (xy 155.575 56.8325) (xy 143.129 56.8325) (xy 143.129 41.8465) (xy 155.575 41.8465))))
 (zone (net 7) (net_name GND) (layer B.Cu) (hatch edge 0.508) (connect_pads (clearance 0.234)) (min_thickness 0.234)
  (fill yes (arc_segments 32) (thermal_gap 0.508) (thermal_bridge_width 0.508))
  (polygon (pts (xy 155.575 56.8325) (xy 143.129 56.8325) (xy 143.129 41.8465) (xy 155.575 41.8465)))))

